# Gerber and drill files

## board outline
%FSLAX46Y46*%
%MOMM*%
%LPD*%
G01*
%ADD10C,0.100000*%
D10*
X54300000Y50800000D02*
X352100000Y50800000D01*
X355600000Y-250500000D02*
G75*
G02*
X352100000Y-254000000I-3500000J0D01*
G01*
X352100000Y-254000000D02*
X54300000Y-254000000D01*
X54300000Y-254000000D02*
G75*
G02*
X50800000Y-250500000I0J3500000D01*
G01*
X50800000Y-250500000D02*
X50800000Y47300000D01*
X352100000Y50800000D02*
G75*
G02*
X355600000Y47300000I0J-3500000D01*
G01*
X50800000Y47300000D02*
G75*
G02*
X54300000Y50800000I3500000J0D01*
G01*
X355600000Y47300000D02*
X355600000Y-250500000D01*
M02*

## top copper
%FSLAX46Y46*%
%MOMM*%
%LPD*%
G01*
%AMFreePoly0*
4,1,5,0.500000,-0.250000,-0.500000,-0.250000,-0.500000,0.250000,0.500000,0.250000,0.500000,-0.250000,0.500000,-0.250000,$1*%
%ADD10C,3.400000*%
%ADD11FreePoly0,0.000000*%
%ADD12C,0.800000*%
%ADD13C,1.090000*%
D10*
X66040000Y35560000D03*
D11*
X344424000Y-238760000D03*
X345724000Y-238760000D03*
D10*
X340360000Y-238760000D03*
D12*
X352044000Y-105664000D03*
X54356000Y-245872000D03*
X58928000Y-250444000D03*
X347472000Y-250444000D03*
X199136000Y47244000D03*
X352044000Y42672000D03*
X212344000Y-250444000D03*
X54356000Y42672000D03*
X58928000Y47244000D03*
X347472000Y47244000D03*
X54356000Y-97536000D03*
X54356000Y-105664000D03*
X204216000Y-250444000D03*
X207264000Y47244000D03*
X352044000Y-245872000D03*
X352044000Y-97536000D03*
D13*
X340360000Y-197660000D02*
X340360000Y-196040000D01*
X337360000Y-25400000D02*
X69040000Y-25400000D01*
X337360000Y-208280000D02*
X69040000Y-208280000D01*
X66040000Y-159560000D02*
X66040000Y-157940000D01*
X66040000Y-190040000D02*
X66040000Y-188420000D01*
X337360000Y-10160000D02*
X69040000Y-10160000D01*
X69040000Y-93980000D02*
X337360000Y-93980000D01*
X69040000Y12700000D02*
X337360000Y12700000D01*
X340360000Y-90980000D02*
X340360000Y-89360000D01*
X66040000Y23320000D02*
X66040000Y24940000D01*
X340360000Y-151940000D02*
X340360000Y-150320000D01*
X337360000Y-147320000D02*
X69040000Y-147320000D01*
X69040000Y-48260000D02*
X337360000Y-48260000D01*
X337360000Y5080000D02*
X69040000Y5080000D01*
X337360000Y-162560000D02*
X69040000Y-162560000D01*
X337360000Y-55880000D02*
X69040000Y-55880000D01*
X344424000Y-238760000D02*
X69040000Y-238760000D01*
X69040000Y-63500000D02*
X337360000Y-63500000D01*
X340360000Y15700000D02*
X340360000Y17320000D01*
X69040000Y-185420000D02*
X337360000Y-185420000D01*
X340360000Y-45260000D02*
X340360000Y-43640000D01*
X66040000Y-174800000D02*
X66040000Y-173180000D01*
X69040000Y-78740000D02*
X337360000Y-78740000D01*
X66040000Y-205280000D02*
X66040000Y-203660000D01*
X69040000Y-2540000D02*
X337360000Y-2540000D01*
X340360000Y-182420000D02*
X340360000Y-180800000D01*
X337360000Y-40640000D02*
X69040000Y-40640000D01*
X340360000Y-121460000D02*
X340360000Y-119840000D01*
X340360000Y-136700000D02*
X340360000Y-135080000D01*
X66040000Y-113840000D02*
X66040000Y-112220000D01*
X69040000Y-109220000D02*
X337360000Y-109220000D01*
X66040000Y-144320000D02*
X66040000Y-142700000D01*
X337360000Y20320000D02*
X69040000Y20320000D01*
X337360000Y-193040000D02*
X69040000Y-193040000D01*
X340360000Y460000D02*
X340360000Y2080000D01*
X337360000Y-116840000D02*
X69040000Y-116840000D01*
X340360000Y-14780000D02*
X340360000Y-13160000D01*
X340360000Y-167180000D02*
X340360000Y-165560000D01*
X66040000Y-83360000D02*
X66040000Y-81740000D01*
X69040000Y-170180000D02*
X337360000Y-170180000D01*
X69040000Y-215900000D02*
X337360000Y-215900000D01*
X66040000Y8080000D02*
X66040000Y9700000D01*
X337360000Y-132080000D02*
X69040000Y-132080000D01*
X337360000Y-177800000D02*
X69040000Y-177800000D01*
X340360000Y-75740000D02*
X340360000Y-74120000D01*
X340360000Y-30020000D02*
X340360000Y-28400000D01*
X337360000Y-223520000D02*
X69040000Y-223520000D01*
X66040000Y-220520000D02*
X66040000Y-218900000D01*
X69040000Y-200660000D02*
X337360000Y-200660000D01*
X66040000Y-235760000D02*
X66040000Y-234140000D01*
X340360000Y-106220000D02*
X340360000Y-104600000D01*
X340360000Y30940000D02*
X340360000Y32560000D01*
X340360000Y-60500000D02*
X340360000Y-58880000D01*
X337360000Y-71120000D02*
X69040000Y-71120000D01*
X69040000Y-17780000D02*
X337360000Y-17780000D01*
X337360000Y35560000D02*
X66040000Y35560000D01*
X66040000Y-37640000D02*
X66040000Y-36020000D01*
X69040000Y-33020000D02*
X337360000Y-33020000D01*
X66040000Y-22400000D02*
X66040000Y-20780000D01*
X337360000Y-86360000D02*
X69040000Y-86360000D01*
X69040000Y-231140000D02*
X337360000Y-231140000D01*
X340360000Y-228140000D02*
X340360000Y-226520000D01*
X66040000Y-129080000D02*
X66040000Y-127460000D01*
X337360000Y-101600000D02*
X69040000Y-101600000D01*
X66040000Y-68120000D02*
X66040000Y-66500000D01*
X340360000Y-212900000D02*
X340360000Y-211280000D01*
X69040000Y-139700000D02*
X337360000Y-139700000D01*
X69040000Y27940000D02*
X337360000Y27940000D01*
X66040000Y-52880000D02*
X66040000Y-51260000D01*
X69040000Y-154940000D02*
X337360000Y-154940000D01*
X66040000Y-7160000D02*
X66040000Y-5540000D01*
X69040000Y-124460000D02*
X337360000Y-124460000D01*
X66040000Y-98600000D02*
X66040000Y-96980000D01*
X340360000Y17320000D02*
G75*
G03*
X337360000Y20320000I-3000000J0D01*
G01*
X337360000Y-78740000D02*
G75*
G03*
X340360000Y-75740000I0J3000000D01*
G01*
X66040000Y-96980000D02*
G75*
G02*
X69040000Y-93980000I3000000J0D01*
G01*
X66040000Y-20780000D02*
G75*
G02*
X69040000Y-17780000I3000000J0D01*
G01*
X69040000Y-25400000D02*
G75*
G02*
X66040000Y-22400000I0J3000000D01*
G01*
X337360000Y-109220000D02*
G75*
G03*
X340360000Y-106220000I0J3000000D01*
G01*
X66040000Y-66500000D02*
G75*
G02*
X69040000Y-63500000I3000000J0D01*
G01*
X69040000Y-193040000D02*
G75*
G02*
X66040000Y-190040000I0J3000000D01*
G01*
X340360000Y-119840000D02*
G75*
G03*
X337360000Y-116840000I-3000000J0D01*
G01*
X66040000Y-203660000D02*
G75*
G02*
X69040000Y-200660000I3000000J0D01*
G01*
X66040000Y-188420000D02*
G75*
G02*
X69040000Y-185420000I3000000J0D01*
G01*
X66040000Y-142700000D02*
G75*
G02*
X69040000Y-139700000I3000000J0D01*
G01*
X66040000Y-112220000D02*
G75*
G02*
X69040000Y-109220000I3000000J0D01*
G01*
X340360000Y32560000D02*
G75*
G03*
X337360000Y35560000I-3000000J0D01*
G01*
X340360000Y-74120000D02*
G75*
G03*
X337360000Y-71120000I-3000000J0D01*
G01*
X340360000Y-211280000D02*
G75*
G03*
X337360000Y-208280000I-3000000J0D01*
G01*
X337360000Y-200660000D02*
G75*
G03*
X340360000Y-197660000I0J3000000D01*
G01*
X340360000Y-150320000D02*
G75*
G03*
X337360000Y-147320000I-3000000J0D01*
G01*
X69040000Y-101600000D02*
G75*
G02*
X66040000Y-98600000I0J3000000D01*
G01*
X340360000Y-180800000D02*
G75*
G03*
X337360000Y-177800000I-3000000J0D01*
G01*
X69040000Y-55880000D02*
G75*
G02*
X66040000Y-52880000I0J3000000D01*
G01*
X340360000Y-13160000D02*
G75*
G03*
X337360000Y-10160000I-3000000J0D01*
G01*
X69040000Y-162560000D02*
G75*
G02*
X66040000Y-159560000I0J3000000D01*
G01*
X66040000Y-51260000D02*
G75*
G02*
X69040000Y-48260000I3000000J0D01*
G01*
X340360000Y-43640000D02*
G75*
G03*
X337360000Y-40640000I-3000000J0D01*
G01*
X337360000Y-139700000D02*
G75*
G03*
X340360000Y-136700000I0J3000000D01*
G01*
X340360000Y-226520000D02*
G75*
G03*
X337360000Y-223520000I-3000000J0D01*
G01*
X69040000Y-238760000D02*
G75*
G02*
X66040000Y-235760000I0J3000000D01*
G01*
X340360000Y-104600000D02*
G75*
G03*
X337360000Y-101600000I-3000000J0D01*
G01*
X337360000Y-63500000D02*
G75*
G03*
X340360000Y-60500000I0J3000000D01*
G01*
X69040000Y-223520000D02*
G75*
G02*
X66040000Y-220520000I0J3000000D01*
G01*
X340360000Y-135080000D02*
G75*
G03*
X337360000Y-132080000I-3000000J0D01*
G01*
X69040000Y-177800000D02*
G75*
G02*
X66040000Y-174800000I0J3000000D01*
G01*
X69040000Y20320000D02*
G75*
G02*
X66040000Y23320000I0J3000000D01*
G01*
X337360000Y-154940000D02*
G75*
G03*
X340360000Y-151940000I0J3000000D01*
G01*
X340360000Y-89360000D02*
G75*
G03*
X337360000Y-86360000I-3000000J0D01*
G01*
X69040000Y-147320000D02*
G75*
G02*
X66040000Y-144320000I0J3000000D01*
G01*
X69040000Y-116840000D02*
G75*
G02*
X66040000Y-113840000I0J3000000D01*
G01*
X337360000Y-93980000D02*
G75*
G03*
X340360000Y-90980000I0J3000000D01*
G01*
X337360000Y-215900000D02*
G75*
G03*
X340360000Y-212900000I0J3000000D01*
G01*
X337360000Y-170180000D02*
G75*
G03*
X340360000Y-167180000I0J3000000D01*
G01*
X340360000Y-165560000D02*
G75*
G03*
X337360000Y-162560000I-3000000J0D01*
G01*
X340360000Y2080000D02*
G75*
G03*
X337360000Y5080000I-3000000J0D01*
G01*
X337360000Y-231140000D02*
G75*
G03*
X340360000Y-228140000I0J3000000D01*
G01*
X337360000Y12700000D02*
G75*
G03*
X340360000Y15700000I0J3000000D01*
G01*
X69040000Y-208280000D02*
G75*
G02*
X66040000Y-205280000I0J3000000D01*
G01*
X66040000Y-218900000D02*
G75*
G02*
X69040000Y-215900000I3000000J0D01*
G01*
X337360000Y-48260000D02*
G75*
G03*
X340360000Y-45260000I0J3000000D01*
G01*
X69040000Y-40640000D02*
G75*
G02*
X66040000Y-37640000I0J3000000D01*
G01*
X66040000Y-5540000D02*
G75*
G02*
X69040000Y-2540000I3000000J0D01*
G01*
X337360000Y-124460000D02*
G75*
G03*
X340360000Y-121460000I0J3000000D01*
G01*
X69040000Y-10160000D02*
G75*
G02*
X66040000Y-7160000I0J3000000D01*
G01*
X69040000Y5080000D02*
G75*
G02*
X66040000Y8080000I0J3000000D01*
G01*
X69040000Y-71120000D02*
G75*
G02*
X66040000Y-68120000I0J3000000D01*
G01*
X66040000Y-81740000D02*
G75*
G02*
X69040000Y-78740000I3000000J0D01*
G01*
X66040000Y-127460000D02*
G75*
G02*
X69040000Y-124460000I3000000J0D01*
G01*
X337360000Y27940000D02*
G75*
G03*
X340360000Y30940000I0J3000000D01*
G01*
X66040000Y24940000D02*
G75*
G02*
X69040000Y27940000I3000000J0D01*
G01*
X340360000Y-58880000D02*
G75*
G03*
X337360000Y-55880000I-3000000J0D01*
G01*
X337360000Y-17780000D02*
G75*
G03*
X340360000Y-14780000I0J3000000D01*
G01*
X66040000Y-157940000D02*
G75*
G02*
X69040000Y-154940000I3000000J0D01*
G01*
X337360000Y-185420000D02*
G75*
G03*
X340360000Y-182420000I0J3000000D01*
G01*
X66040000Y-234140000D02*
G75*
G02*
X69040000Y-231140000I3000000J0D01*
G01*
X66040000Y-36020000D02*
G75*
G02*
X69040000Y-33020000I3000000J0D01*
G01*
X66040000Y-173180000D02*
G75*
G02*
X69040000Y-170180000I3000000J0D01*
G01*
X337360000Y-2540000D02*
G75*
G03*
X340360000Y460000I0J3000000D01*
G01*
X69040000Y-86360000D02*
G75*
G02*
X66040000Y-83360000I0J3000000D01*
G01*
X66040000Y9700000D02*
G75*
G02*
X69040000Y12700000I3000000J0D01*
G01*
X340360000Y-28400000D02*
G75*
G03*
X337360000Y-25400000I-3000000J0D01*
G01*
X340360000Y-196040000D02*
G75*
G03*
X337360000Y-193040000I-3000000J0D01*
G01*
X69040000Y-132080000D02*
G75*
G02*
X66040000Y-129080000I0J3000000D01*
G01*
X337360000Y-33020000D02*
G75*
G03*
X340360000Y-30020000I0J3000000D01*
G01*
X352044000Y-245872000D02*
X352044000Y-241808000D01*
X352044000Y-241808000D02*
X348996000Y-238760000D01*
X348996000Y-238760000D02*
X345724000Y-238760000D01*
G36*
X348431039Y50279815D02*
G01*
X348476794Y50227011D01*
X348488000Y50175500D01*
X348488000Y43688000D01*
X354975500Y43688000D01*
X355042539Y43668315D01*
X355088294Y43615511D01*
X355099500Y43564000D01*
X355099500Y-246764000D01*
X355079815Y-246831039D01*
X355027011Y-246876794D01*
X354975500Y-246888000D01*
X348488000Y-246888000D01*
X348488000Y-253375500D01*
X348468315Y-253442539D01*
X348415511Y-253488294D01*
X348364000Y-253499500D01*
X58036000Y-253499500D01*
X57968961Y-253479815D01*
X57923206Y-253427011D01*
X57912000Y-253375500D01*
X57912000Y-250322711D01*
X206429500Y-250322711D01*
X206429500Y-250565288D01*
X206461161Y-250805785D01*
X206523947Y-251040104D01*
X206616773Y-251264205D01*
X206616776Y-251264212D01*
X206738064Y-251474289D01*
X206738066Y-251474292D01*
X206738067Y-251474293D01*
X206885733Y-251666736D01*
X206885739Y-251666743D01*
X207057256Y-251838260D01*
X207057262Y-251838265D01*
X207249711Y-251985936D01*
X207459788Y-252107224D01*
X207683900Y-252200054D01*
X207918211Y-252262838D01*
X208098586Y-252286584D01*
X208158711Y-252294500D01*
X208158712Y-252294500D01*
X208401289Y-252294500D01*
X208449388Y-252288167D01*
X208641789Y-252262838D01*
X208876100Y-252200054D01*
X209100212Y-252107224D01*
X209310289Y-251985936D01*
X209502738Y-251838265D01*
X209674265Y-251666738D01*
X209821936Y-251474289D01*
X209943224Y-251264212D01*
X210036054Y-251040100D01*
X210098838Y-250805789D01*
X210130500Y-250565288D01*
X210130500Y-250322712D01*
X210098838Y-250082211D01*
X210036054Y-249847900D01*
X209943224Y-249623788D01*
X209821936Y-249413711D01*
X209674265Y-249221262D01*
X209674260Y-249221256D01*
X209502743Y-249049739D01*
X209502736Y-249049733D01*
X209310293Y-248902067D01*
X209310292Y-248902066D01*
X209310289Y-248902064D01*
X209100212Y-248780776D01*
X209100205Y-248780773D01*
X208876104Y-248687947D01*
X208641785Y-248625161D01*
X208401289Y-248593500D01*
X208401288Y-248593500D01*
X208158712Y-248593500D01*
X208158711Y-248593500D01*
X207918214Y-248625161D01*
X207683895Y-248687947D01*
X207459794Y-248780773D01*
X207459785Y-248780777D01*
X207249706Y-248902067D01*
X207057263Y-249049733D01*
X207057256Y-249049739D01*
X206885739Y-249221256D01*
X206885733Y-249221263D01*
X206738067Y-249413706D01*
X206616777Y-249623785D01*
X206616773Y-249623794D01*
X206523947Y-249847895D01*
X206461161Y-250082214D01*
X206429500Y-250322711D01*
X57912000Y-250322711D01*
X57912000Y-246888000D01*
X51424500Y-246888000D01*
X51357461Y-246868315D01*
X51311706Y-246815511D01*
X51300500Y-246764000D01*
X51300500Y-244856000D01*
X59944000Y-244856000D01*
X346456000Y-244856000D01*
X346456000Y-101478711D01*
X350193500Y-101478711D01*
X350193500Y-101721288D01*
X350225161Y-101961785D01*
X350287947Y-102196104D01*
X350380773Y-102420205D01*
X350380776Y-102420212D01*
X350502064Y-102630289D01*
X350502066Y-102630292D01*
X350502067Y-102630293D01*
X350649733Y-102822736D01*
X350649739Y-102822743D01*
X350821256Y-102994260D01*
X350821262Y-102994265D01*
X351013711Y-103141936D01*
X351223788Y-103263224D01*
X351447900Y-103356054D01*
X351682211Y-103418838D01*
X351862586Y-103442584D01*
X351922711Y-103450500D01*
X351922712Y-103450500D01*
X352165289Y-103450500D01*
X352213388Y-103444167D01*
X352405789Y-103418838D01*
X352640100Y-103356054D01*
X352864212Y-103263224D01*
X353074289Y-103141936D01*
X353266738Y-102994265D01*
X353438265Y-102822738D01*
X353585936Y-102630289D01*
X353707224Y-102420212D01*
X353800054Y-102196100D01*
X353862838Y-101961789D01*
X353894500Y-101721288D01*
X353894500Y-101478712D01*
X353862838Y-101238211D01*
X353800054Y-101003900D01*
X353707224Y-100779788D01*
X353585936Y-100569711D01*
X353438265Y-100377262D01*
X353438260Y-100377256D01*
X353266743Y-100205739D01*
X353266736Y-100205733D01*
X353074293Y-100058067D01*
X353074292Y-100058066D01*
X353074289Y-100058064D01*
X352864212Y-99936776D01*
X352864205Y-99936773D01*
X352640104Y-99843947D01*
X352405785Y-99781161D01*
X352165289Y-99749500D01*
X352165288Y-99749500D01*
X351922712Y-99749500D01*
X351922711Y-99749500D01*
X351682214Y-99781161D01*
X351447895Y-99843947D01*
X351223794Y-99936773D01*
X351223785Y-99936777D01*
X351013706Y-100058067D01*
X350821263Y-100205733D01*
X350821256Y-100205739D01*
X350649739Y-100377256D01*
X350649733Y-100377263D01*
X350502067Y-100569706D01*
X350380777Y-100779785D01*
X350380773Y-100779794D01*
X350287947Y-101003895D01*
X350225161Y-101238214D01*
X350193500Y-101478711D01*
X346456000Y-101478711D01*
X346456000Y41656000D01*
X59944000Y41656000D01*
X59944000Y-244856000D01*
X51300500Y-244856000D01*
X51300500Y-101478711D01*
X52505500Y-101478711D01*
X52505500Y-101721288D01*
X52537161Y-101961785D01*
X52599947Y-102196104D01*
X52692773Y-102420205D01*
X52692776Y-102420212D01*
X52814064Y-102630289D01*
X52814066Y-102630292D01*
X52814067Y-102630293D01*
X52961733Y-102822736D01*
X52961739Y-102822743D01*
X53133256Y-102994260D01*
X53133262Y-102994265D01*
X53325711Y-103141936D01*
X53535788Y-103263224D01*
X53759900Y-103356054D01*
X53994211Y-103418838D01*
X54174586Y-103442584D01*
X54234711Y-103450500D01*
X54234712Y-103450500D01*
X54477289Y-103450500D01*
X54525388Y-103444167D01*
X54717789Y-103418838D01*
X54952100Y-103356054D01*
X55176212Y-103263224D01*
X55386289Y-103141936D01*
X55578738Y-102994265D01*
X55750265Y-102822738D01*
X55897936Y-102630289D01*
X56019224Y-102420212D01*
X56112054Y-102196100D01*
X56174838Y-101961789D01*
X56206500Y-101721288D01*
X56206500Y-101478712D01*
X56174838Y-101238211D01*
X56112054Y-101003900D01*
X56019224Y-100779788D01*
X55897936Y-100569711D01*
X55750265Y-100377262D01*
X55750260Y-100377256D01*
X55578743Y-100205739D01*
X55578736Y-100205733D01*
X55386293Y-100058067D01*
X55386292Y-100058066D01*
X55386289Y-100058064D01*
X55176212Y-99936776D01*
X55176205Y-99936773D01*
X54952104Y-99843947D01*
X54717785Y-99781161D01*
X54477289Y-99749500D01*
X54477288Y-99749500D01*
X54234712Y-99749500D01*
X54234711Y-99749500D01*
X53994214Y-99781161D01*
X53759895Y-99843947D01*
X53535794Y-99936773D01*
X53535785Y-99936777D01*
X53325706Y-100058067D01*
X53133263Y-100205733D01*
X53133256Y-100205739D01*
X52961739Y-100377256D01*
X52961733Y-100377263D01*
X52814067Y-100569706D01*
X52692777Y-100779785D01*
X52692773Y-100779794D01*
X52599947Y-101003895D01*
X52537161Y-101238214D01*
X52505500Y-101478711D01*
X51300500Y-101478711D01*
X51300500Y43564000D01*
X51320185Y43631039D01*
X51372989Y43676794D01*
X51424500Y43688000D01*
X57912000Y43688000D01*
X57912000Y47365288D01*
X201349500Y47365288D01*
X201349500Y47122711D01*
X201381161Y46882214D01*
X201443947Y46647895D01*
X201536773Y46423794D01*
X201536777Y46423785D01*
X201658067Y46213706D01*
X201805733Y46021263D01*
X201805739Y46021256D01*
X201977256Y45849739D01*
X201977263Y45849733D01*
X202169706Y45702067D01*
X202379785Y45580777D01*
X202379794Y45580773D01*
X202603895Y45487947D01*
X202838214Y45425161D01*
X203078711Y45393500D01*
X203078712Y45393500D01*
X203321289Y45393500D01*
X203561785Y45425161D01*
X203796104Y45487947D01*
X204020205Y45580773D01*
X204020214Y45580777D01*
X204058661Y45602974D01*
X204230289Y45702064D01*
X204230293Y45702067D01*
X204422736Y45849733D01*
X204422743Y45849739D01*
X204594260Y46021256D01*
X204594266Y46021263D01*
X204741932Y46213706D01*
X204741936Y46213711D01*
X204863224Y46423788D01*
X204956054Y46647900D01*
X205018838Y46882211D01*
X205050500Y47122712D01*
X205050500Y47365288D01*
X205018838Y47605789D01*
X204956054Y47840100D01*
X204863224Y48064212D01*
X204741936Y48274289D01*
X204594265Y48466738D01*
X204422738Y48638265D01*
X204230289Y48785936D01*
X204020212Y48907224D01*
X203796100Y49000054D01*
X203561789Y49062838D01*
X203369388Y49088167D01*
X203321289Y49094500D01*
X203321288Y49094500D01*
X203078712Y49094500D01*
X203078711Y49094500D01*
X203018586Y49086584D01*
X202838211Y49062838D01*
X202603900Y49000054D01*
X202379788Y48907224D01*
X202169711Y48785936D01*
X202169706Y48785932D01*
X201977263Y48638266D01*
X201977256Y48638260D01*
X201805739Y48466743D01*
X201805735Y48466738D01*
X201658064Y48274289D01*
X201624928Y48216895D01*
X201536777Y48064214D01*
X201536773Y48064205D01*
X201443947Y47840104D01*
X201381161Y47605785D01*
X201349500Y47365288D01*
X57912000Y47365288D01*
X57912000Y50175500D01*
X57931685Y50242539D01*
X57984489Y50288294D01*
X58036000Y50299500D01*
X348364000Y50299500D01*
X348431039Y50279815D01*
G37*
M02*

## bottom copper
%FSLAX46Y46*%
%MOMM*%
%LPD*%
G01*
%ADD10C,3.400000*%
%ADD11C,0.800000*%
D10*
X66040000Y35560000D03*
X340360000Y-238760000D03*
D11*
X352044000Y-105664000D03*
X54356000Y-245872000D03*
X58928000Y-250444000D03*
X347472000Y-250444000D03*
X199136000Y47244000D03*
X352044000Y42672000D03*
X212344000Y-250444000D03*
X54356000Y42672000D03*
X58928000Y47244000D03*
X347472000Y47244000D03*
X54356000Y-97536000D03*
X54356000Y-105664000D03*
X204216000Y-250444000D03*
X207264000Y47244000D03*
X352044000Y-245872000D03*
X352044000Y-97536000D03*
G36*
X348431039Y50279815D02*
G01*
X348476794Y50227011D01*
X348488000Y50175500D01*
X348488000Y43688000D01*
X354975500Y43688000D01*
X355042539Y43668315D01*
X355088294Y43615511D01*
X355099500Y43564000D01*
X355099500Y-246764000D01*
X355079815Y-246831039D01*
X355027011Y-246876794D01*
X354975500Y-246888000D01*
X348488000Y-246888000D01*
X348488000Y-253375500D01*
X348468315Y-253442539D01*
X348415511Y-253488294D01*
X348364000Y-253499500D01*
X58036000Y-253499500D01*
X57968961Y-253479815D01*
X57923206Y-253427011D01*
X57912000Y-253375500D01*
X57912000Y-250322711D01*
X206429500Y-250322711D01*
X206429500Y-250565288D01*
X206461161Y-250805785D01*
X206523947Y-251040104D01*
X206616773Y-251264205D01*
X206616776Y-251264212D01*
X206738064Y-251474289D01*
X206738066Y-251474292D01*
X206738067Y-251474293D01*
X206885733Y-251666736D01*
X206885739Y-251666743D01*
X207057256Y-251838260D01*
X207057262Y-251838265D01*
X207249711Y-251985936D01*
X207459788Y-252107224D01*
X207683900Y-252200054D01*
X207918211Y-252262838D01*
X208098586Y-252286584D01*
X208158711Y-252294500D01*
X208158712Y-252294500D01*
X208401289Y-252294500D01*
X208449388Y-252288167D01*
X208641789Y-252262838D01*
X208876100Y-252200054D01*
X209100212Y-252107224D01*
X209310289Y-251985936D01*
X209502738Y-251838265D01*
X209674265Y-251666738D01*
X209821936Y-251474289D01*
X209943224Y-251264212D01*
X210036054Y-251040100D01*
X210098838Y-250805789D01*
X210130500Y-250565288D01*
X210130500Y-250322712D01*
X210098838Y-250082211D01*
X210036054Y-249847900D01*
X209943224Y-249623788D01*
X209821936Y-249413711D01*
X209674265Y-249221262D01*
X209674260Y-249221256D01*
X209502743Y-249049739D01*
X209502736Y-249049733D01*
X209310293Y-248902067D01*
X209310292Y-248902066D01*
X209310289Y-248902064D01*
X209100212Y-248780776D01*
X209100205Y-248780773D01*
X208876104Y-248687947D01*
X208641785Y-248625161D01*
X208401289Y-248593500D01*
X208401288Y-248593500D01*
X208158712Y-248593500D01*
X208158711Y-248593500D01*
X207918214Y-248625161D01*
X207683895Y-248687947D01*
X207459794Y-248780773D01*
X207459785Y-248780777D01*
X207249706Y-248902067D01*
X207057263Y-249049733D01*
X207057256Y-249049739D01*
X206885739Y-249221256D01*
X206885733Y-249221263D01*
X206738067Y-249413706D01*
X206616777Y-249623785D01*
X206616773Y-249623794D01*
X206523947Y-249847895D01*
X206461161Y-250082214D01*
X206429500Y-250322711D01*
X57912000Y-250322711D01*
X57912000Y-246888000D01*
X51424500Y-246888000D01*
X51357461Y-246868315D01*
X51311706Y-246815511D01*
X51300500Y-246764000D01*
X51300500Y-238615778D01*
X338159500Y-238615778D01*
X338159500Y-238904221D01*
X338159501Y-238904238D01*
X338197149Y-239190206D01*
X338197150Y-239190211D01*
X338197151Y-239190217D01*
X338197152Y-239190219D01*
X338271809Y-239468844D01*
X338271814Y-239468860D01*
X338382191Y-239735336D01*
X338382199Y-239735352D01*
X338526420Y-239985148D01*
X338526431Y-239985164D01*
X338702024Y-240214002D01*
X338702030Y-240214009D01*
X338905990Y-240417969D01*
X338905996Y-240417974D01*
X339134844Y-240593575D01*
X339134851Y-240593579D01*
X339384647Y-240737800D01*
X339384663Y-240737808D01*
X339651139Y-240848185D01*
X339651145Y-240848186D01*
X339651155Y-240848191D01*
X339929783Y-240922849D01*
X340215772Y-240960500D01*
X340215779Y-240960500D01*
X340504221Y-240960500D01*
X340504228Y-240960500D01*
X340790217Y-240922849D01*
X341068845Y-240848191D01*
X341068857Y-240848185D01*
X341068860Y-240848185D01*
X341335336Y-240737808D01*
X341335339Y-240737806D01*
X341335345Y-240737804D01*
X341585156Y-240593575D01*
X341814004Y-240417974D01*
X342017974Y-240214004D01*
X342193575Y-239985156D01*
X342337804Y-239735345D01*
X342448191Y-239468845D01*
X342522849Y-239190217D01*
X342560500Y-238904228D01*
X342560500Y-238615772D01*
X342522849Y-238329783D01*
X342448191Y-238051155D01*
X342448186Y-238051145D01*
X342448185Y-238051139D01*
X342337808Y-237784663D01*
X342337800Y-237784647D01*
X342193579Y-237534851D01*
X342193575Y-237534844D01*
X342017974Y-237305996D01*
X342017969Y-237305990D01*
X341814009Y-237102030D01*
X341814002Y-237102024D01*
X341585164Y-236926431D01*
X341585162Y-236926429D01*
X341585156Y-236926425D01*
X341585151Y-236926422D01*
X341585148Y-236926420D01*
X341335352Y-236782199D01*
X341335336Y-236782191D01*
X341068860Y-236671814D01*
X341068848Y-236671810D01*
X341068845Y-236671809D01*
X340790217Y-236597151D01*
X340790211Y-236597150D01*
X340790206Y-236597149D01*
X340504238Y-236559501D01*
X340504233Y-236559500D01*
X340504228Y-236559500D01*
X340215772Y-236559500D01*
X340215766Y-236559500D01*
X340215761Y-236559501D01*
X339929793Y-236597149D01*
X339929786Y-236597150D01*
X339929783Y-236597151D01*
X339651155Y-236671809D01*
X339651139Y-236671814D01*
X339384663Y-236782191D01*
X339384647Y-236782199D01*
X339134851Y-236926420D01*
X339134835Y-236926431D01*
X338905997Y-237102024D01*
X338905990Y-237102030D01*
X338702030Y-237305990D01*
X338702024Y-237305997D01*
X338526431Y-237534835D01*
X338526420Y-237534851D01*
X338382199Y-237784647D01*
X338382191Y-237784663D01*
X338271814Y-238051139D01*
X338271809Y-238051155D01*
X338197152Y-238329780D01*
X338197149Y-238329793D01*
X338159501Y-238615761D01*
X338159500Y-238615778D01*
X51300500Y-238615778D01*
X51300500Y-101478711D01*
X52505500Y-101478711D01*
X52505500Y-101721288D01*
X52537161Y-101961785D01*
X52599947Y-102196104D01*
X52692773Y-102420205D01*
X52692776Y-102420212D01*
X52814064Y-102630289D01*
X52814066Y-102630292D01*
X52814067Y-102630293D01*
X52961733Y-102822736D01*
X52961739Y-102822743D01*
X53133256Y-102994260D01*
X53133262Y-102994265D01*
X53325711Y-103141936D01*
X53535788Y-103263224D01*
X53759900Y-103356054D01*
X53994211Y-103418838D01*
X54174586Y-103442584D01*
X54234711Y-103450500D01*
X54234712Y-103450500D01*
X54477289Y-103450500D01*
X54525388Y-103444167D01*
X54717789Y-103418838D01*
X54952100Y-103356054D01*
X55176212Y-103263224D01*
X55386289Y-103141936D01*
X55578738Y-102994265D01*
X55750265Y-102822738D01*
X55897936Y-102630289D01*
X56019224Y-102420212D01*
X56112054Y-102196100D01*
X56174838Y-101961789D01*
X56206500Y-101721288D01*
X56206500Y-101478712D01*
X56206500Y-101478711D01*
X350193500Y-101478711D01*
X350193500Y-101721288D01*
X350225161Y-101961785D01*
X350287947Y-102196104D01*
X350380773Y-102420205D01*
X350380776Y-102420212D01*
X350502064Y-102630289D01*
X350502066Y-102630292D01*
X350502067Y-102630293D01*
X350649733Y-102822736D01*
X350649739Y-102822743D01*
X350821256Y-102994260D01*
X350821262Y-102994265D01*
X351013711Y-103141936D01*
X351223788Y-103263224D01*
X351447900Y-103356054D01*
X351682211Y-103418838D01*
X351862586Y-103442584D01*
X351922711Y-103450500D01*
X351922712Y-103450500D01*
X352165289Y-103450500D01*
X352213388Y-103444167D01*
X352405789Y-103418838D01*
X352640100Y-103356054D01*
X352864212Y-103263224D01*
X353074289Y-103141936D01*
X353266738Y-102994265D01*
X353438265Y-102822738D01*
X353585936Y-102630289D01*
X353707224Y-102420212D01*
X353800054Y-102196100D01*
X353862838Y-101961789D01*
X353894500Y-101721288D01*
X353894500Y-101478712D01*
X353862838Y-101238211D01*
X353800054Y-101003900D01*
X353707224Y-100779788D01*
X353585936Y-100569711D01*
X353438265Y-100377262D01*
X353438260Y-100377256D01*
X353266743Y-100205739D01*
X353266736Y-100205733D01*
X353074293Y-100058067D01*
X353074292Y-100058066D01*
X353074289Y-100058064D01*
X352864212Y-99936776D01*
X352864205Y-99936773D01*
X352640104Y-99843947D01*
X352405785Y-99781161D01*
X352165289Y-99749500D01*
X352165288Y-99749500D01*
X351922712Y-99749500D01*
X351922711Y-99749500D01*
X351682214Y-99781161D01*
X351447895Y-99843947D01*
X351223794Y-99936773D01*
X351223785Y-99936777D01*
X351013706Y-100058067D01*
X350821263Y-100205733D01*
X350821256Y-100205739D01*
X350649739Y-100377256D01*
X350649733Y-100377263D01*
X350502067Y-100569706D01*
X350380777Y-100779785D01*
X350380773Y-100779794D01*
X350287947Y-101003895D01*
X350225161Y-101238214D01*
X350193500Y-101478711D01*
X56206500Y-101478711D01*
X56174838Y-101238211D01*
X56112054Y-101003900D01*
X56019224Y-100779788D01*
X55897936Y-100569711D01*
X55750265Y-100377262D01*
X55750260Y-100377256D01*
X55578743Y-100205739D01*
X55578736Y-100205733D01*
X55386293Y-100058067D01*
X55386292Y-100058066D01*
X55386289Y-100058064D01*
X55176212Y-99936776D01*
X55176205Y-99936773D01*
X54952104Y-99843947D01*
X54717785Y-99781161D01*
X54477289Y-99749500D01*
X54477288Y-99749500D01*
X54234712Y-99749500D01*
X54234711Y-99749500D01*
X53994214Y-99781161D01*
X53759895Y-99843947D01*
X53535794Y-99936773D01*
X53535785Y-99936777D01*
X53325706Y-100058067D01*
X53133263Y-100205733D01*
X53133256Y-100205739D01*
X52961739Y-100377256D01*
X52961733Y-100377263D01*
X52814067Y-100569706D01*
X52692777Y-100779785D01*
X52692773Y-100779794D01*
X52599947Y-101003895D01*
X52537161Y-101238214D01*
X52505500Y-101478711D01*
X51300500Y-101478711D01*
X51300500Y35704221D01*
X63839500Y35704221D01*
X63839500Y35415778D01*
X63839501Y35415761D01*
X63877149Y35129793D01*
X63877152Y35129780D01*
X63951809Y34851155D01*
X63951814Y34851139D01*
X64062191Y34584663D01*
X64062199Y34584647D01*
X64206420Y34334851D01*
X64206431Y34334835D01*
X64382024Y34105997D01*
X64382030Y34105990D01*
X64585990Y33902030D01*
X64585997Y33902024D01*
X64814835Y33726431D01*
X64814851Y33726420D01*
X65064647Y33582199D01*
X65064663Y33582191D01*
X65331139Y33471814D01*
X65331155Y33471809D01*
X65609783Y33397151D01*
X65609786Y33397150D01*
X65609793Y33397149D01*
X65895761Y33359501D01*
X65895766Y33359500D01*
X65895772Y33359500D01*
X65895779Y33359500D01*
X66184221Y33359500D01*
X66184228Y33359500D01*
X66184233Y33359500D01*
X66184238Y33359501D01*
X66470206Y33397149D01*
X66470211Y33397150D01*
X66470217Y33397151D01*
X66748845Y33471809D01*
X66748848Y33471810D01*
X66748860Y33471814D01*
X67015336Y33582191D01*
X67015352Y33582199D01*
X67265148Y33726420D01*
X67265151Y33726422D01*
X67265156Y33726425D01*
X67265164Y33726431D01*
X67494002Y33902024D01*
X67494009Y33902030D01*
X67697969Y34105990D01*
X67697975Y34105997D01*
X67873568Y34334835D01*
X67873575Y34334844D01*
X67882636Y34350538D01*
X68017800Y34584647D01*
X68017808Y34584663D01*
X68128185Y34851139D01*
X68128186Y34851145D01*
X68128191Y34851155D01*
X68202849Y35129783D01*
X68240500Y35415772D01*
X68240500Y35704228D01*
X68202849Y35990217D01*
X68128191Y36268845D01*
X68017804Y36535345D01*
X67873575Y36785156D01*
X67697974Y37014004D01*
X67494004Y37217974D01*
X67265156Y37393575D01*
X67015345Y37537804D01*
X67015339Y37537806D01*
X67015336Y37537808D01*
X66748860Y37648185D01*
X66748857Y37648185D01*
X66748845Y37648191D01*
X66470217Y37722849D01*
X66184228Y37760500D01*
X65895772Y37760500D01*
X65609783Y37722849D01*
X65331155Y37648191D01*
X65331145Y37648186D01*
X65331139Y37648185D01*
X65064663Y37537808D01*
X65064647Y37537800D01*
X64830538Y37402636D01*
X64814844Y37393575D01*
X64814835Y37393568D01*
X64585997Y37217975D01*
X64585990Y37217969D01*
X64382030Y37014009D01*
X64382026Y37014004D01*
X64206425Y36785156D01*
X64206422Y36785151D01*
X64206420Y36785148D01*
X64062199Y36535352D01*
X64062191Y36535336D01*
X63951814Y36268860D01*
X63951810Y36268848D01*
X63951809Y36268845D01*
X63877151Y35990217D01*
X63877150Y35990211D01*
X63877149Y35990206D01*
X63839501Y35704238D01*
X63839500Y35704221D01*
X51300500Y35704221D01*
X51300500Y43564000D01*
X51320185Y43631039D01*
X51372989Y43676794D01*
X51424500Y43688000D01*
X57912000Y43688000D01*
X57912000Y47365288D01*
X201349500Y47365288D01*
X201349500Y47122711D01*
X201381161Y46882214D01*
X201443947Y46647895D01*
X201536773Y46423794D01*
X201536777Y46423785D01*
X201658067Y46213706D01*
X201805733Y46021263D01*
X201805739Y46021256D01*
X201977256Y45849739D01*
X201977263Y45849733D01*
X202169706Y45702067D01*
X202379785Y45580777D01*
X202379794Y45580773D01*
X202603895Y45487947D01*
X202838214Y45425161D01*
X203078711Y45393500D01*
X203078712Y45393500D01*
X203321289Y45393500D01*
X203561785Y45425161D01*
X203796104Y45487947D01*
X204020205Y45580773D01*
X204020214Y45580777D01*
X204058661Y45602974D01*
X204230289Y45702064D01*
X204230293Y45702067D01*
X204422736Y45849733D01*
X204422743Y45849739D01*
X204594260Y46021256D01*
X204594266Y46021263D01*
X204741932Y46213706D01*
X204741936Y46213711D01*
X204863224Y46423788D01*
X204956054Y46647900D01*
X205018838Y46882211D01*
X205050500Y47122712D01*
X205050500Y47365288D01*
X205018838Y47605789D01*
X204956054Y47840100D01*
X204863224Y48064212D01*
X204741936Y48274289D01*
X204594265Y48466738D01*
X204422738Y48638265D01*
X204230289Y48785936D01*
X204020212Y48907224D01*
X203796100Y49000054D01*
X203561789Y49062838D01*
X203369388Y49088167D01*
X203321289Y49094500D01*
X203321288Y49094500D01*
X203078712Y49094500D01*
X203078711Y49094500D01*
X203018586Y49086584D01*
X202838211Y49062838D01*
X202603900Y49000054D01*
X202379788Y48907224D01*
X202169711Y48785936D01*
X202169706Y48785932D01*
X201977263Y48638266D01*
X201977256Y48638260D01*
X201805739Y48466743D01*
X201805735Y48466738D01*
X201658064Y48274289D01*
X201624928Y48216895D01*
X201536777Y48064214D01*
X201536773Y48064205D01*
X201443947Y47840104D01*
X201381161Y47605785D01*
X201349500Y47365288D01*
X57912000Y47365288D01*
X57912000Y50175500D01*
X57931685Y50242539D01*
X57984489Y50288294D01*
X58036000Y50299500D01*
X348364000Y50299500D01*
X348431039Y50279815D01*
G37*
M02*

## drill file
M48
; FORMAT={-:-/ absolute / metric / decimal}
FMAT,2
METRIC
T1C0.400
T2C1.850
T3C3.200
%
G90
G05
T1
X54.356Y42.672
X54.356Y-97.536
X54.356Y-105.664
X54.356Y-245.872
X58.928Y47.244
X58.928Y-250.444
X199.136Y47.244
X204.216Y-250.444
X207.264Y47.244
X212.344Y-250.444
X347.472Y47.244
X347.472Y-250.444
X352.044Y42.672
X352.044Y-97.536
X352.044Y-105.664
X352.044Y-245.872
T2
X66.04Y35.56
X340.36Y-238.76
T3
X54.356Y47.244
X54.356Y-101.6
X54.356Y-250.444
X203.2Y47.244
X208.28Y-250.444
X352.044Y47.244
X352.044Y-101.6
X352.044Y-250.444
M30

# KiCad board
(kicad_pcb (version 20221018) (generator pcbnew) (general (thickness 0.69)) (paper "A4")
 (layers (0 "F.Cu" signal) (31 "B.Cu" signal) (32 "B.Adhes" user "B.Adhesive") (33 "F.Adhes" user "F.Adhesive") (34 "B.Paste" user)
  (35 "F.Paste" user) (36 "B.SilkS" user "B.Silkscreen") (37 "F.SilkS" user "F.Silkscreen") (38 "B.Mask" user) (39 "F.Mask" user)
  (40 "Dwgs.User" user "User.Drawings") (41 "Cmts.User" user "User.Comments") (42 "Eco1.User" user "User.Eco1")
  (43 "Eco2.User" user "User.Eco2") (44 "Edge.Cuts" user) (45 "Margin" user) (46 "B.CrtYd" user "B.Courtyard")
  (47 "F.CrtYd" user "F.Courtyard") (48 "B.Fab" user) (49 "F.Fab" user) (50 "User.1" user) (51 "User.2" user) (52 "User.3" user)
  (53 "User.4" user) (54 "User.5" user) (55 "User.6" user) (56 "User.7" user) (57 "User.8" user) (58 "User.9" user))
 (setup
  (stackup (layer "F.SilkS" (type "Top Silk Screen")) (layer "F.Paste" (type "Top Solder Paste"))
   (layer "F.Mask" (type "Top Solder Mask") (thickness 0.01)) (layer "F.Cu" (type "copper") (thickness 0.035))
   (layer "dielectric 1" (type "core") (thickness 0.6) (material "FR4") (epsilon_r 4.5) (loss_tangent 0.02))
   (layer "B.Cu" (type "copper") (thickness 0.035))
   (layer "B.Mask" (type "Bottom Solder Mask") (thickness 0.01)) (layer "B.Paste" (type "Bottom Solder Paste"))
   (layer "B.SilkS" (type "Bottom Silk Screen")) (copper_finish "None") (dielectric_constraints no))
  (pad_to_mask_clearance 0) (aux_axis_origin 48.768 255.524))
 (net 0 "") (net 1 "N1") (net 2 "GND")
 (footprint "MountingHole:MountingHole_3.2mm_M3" (layer "F.Cu") (at 203.2 -47.244)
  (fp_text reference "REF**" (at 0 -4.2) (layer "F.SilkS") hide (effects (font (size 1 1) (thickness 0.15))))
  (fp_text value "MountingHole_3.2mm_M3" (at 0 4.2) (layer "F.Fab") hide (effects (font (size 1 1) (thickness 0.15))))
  (pad "" np_thru_hole circle (at 0 0) (size 3.2 3.2) (drill 3.2) (layers "F&B.Cu" "*.Mask")))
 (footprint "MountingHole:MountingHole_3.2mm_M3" (layer "F.Cu") (at 208.28 250.444)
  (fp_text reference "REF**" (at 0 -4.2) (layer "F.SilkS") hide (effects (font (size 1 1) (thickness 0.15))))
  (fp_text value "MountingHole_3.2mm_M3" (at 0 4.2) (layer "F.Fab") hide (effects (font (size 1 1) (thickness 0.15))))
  (pad "" np_thru_hole circle (at 0 0) (size 3.2 3.2) (drill 3.2) (layers "F&B.Cu" "*.Mask")))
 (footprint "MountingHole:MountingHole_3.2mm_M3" (layer "F.Cu") (at 54.356 101.6)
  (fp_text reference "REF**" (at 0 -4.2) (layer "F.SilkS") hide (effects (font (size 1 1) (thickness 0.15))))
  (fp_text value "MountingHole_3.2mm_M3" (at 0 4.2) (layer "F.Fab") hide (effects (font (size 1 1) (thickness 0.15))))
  (pad "" np_thru_hole circle (at 0 0) (size 3.2 3.2) (drill 3.2) (layers "F&B.Cu" "*.Mask")))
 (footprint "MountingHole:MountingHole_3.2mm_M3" (layer "F.Cu") (at 352.044 250.444)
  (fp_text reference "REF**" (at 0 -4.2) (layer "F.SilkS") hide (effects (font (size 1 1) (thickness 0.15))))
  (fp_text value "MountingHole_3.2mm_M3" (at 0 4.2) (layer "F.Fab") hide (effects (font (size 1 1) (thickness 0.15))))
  (pad "" np_thru_hole circle (at 0 0) (size 3.2 3.2) (drill 3.2) (layers "F&B.Cu" "*.Mask")))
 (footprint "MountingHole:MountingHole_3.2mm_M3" (layer "F.Cu") (at 54.356 250.444)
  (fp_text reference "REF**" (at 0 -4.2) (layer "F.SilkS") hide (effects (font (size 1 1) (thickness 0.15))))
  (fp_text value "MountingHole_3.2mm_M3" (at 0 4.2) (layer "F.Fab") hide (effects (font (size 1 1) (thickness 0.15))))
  (pad "" np_thru_hole circle (at 0 0) (size 3.2 3.2) (drill 3.2) (layers "F&B.Cu" "*.Mask")))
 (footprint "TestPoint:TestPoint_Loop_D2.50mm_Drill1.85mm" (layer "F.Cu") (at 66.04 -35.56)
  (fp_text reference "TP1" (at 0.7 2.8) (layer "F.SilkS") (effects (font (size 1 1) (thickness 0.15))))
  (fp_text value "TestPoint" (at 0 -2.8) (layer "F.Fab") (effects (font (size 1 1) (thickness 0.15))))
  (pad "1" thru_hole circle (at 0 0) (size 3.4 3.4) (drill 1.85) (layers "*.Cu" "*.Mask") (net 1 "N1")))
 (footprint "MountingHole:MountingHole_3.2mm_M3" (layer "F.Cu") (at 352.044 -47.244)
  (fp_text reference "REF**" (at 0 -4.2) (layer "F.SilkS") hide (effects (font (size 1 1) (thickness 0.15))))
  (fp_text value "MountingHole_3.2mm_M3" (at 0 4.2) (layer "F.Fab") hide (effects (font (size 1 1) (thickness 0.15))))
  (pad "" np_thru_hole circle (at 0 0) (size 3.2 3.2) (drill 3.2) (layers "F&B.Cu" "*.Mask")))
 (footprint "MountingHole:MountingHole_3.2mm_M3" (layer "F.Cu") (at 54.356 -47.244)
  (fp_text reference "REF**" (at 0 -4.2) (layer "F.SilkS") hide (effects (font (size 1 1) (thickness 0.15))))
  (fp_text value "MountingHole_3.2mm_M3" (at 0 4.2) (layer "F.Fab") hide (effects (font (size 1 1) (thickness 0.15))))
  (pad "" np_thru_hole circle (at 0 0) (size 3.2 3.2) (drill 3.2) (layers "*.Cu" "*.Mask")))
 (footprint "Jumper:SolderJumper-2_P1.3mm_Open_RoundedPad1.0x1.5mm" (layer "F.Cu") (at 345.074 238.76)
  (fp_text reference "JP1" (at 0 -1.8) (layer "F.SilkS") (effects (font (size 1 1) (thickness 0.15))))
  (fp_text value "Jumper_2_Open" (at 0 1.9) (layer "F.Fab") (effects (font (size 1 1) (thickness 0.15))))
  (pad "1" smd custom (at -0.65 0) (size 1 0.5) (layers "F.Cu" "F.Mask") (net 1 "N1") (zone_connect 2) (thermal_bridge_angle 45)
   (options (clearance outline) (anchor rect)) (primitives))
  (pad "2" smd custom (at 0.65 0) (size 1 0.5) (layers "F.Cu" "F.Mask") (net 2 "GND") (zone_connect 2) (thermal_bridge_angle 45)
   (options (clearance outline) (anchor rect)) (primitives)))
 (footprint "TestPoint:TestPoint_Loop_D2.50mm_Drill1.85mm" (layer "F.Cu") (at 340.36 238.76)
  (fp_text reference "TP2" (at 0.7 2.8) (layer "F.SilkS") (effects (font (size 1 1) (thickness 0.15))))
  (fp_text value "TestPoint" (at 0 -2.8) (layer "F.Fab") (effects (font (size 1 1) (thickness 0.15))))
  (pad "1" thru_hole circle (at 0 0) (size 3.4 3.4) (drill 1.85) (layers "*.Cu" "*.Mask") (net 1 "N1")))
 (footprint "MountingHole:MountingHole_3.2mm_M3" (layer "F.Cu") (at 352.044 101.6)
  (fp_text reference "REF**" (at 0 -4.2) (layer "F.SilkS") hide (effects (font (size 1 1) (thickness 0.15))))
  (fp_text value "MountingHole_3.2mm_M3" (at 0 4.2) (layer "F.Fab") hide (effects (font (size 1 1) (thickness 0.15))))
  (pad "" np_thru_hole circle (at 0 0) (size 3.2 3.2) (drill 3.2) (layers "F&B.Cu" "*.Mask")))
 (gr_line (start 54.3 -50.8) (end 352.1 -50.8) (stroke (width 0.1) (type default)) (layer "Edge.Cuts"))
 (gr_arc (start 355.6 250.5) (mid 354.574874 252.974874) (end 352.1 254) (stroke (width 0.1) (type default)) (layer "Edge.Cuts"))
 (gr_line (start 352.1 254) (end 54.3 254) (stroke (width 0.1) (type default)) (layer "Edge.Cuts"))
 (gr_arc (start 54.3 254) (mid 51.825126 252.974874) (end 50.8 250.5) (stroke (width 0.1) (type default)) (layer "Edge.Cuts"))
 (gr_line (start 50.8 250.5) (end 50.8 -47.3) (stroke (width 0.1) (type default)) (layer "Edge.Cuts"))
 (gr_arc (start 352.1 -50.8) (mid 354.574874 -49.774874) (end 355.6 -47.3) (stroke (width 0.1) (type default)) (layer "Edge.Cuts"))
 (gr_arc (start 50.8 -47.3) (mid 51.825126 -49.774874) (end 54.3 -50.8) (stroke (width 0.1) (type default)) (layer "Edge.Cuts"))
 (gr_line (start 355.6 -47.3) (end 355.6 250.5) (stroke (width 0.1) (type default)) (layer "Edge.Cuts"))
 (segment (start 340.36 197.66) (end 340.36 196.04) (width 1.09) (layer "F.Cu") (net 1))
 (segment (start 337.36 25.4) (end 69.04 25.4) (width 1.09) (layer "F.Cu") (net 1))
 (segment (start 337.36 208.28) (end 69.04 208.28) (width 1.09) (layer "F.Cu") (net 1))
 (segment (start 66.04 159.56) (end 66.04 157.94) (width 1.09) (layer "F.Cu") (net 1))
 (segment (start 66.04 190.04) (end 66.04 188.42) (width 1.09) (layer "F.Cu") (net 1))
 (segment (start 337.36 10.16) (end 69.04 10.16) (width 1.09) (layer "F.Cu") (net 1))
 (segment (start 69.04 93.98) (end 337.36 93.98) (width 1.09) (layer "F.Cu") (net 1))
 (segment (start 69.04 -12.7) (end 337.36 -12.7) (width 1.09) (layer "F.Cu") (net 1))
 (segment (start 340.36 90.98) (end 340.36 89.36) (width 1.09) (layer "F.Cu") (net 1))
 (segment (start 66.04 -23.32) (end 66.04 -24.94) (width 1.09) (layer "F.Cu") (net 1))
 (segment (start 340.36 151.94) (end 340.36 150.32) (width 1.09) (layer "F.Cu") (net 1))
 (segment (start 337.36 147.32) (end 69.04 147.32) (width 1.09) (layer "F.Cu") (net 1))
 (segment (start 69.04 48.26) (end 337.36 48.26) (width 1.09) (layer "F.Cu") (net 1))
 (segment (start 337.36 -5.08) (end 69.04 -5.08) (width 1.09) (layer "F.Cu") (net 1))
 (segment (start 337.36 162.56) (end 69.04 162.56) (width 1.09) (layer "F.Cu") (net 1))
 (segment (start 337.36 55.88) (end 69.04 55.88) (width 1.09) (layer "F.Cu") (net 1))
 (segment (start 344.424 238.76) (end 69.04 238.76) (width 1.09) (layer "F.Cu") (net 1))
 (segment (start 69.04 63.5) (end 337.36 63.5) (width 1.09) (layer "F.Cu") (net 1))
 (segment (start 340.36 -15.7) (end 340.36 -17.32) (width 1.09) (layer "F.Cu") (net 1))
 (segment (start 69.04 185.42) (end 337.36 185.42) (width 1.09) (layer "F.Cu") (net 1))
 (segment (start 340.36 45.26) (end 340.36 43.64) (width 1.09) (layer "F.Cu") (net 1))
 (segment (start 66.04 174.8) (end 66.04 173.18) (width 1.09) (layer "F.Cu") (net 1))
 (segment (start 69.04 78.74) (end 337.36 78.74) (width 1.09) (layer "F.Cu") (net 1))
 (segment (start 66.04 205.28) (end 66.04 203.66) (width 1.09) (layer "F.Cu") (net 1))
 (segment (start 69.04 2.54) (end 337.36 2.54) (width 1.09) (layer "F.Cu") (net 1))
 (segment (start 340.36 182.42) (end 340.36 180.8) (width 1.09) (layer "F.Cu") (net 1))
 (segment (start 337.36 40.64) (end 69.04 40.64) (width 1.09) (layer "F.Cu") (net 1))
 (segment (start 340.36 121.46) (end 340.36 119.84) (width 1.09) (layer "F.Cu") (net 1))
 (segment (start 340.36 136.7) (end 340.36 135.08) (width 1.09) (layer "F.Cu") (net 1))
 (segment (start 66.04 113.84) (end 66.04 112.22) (width 1.09) (layer "F.Cu") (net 1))
 (segment (start 69.04 109.22) (end 337.36 109.22) (width 1.09) (layer "F.Cu") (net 1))
 (segment (start 66.04 144.32) (end 66.04 142.7) (width 1.09) (layer "F.Cu") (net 1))
 (segment (start 337.36 -20.32) (end 69.04 -20.32) (width 1.09) (layer "F.Cu") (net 1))
 (segment (start 337.36 193.04) (end 69.04 193.04) (width 1.09) (layer "F.Cu") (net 1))
 (segment (start 340.36 -0.46) (end 340.36 -2.08) (width 1.09) (layer "F.Cu") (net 1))
 (segment (start 337.36 116.84) (end 69.04 116.84) (width 1.09) (layer "F.Cu") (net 1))
 (segment (start 340.36 14.78) (end 340.36 13.16) (width 1.09) (layer "F.Cu") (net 1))
 (segment (start 340.36 167.18) (end 340.36 165.56) (width 1.09) (layer "F.Cu") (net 1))
 (segment (start 66.04 83.36) (end 66.04 81.74) (width 1.09) (layer "F.Cu") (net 1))
 (segment (start 69.04 170.18) (end 337.36 170.18) (width 1.09) (layer "F.Cu") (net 1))
 (segment (start 69.04 215.9) (end 337.36 215.9) (width 1.09) (layer "F.Cu") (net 1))
 (segment (start 66.04 -8.08) (end 66.04 -9.7) (width 1.09) (layer "F.Cu") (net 1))
 (segment (start 337.36 132.08) (end 69.04 132.08) (width 1.09) (layer "F.Cu") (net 1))
 (segment (start 337.36 177.8) (end 69.04 177.8) (width 1.09) (layer "F.Cu") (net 1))
 (segment (start 340.36 75.74) (end 340.36 74.12) (width 1.09) (layer "F.Cu") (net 1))
 (segment (start 340.36 30.02) (end 340.36 28.4) (width 1.09) (layer "F.Cu") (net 1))
 (segment (start 337.36 223.52) (end 69.04 223.52) (width 1.09) (layer "F.Cu") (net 1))
 (segment (start 66.04 220.52) (end 66.04 218.9) (width 1.09) (layer "F.Cu") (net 1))
 (segment (start 69.04 200.66) (end 337.36 200.66) (width 1.09) (layer "F.Cu") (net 1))
 (segment (start 66.04 235.76) (end 66.04 234.14) (width 1.09) (layer "F.Cu") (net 1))
 (segment (start 340.36 106.22) (end 340.36 104.6) (width 1.09) (layer "F.Cu") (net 1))
 (segment (start 340.36 -30.94) (end 340.36 -32.56) (width 1.09) (layer "F.Cu") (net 1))
 (segment (start 340.36 60.5) (end 340.36 58.88) (width 1.09) (layer "F.Cu") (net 1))
 (segment (start 337.36 71.12) (end 69.04 71.12) (width 1.09) (layer "F.Cu") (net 1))
 (segment (start 69.04 17.78) (end 337.36 17.78) (width 1.09) (layer "F.Cu") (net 1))
 (segment (start 337.36 -35.56) (end 66.04 -35.56) (width 1.09) (layer "F.Cu") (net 1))
 (segment (start 66.04 37.64) (end 66.04 36.02) (width 1.09) (layer "F.Cu") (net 1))
 (segment (start 69.04 33.02) (end 337.36 33.02) (width 1.09) (layer "F.Cu") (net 1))
 (segment (start 66.04 22.4) (end 66.04 20.78) (width 1.09) (layer "F.Cu") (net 1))
 (segment (start 337.36 86.36) (end 69.04 86.36) (width 1.09) (layer "F.Cu") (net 1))
 (segment (start 69.04 231.14) (end 337.36 231.14) (width 1.09) (layer "F.Cu") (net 1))
 (segment (start 340.36 228.14) (end 340.36 226.52) (width 1.09) (layer "F.Cu") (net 1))
 (segment (start 66.04 129.08) (end 66.04 127.46) (width 1.09) (layer "F.Cu") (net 1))
 (segment (start 337.36 101.6) (end 69.04 101.6) (width 1.09) (layer "F.Cu") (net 1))
 (segment (start 66.04 68.12) (end 66.04 66.5) (width 1.09) (layer "F.Cu") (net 1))
 (segment (start 340.36 212.9) (end 340.36 211.28) (width 1.09) (layer "F.Cu") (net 1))
 (segment (start 69.04 139.7) (end 337.36 139.7) (width 1.09) (layer "F.Cu") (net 1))
 (segment (start 69.04 -27.94) (end 337.36 -27.94) (width 1.09) (layer "F.Cu") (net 1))
 (segment (start 66.04 52.88) (end 66.04 51.26) (width 1.09) (layer "F.Cu") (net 1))
 (segment (start 69.04 154.94) (end 337.36 154.94) (width 1.09) (layer "F.Cu") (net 1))
 (segment (start 66.04 7.16) (end 66.04 5.54) (width 1.09) (layer "F.Cu") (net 1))
 (segment (start 69.04 124.46) (end 337.36 124.46) (width 1.09) (layer "F.Cu") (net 1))
 (segment (start 66.04 98.6) (end 66.04 96.98) (width 1.09) (layer "F.Cu") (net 1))
 (arc (start 340.36 -17.32) (mid 339.48132 -19.44132) (end 337.36 -20.32) (width 1.09) (layer "F.Cu") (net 1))
 (arc (start 337.36 78.74) (mid 339.48132 77.86132) (end 340.36 75.74) (width 1.09) (layer "F.Cu") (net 1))
 (arc (start 66.04 96.98) (mid 66.91868 94.85868) (end 69.04 93.98) (width 1.09) (layer "F.Cu") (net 1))
 (arc (start 66.04 20.78) (mid 66.91868 18.65868) (end 69.04 17.78) (width 1.09) (layer "F.Cu") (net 1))
 (arc (start 69.04 25.4) (mid 66.91868 24.52132) (end 66.04 22.4) (width 1.09) (layer "F.Cu") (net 1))
 (arc (start 337.36 109.22) (mid 339.48132 108.34132) (end 340.36 106.22) (width 1.09) (layer "F.Cu") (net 1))
 (arc (start 66.04 66.5) (mid 66.91868 64.37868) (end 69.04 63.5) (width 1.09) (layer "F.Cu") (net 1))
 (arc (start 69.04 193.04) (mid 66.91868 192.16132) (end 66.04 190.04) (width 1.09) (layer "F.Cu") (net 1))
 (arc (start 340.36 119.84) (mid 339.48132 117.71868) (end 337.36 116.84) (width 1.09) (layer "F.Cu") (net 1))
 (arc (start 66.04 203.66) (mid 66.91868 201.53868) (end 69.04 200.66) (width 1.09) (layer "F.Cu") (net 1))
 (arc (start 66.04 188.42) (mid 66.91868 186.29868) (end 69.04 185.42) (width 1.09) (layer "F.Cu") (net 1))
 (arc (start 66.04 142.7) (mid 66.91868 140.57868) (end 69.04 139.7) (width 1.09) (layer "F.Cu") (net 1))
 (arc (start 66.04 112.22) (mid 66.91868 110.09868) (end 69.04 109.22) (width 1.09) (layer "F.Cu") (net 1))
 (arc (start 340.36 -32.56) (mid 339.48132 -34.68132) (end 337.36 -35.56) (width 1.09) (layer "F.Cu") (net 1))
 (arc (start 340.36 74.12) (mid 339.48132 71.99868) (end 337.36 71.12) (width 1.09) (layer "F.Cu") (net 1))
 (arc (start 340.36 211.28) (mid 339.48132 209.15868) (end 337.36 208.28) (width 1.09) (layer "F.Cu") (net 1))
 (arc (start 337.36 200.66) (mid 339.48132 199.78132) (end 340.36 197.66) (width 1.09) (layer "F.Cu") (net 1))
 (arc (start 340.36 150.32) (mid 339.48132 148.19868) (end 337.36 147.32) (width 1.09) (layer "F.Cu") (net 1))
 (arc (start 69.04 101.6) (mid 66.91868 100.72132) (end 66.04 98.6) (width 1.09) (layer "F.Cu") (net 1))
 (arc (start 340.36 180.8) (mid 339.48132 178.67868) (end 337.36 177.8) (width 1.09) (layer "F.Cu") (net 1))
 (arc (start 69.04 55.88) (mid 66.91868 55.00132) (end 66.04 52.88) (width 1.09) (layer "F.Cu") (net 1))
 (arc (start 340.36 13.16) (mid 339.48132 11.03868) (end 337.36 10.16) (width 1.09) (layer "F.Cu") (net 1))
 (arc (start 69.04 162.56) (mid 66.91868 161.68132) (end 66.04 159.56) (width 1.09) (layer "F.Cu") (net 1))
 (arc (start 66.04 51.26) (mid 66.91868 49.13868) (end 69.04 48.26) (width 1.09) (layer "F.Cu") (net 1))
 (arc (start 340.36 43.64) (mid 339.48132 41.51868) (end 337.36 40.64) (width 1.09) (layer "F.Cu") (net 1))
 (arc (start 337.36 139.7) (mid 339.48132 138.82132) (end 340.36 136.7) (width 1.09) (layer "F.Cu") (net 1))
 (arc (start 340.36 226.52) (mid 339.48132 224.39868) (end 337.36 223.52) (width 1.09) (layer "F.Cu") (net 1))
 (arc (start 69.04 238.76) (mid 66.91868 237.88132) (end 66.04 235.76) (width 1.09) (layer "F.Cu") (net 1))
 (arc (start 340.36 104.6) (mid 339.48132 102.47868) (end 337.36 101.6) (width 1.09) (layer "F.Cu") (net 1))
 (arc (start 337.36 63.5) (mid 339.48132 62.62132) (end 340.36 60.5) (width 1.09) (layer "F.Cu") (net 1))
 (arc (start 69.04 223.52) (mid 66.91868 222.64132) (end 66.04 220.52) (width 1.09) (layer "F.Cu") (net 1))
 (arc (start 340.36 135.08) (mid 339.48132 132.95868) (end 337.36 132.08) (width 1.09) (layer "F.Cu") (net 1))
 (arc (start 69.04 177.8) (mid 66.91868 176.92132) (end 66.04 174.8) (width 1.09) (layer "F.Cu") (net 1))
 (arc (start 69.04 -20.32) (mid 66.91868 -21.19868) (end 66.04 -23.32) (width 1.09) (layer "F.Cu") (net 1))
 (arc (start 337.36 154.94) (mid 339.48132 154.06132) (end 340.36 151.94) (width 1.09) (layer "F.Cu") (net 1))
 (arc (start 340.36 89.36) (mid 339.48132 87.23868) (end 337.36 86.36) (width 1.09) (layer "F.Cu") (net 1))
 (arc (start 69.04 147.32) (mid 66.91868 146.44132) (end 66.04 144.32) (width 1.09) (layer "F.Cu") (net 1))
 (arc (start 69.04 116.84) (mid 66.91868 115.96132) (end 66.04 113.84) (width 1.09) (layer "F.Cu") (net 1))
 (arc (start 337.36 93.98) (mid 339.48132 93.10132) (end 340.36 90.98) (width 1.09) (layer "F.Cu") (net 1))
 (arc (start 337.36 215.9) (mid 339.48132 215.02132) (end 340.36 212.9) (width 1.09) (layer "F.Cu") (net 1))
 (arc (start 337.36 170.18) (mid 339.48132 169.30132) (end 340.36 167.18) (width 1.09) (layer "F.Cu") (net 1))
 (arc (start 340.36 165.56) (mid 339.48132 163.43868) (end 337.36 162.56) (width 1.09) (layer "F.Cu") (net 1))
 (arc (start 340.36 -2.08) (mid 339.48132 -4.20132) (end 337.36 -5.08) (width 1.09) (layer "F.Cu") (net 1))
 (arc (start 337.36 231.14) (mid 339.48132 230.26132) (end 340.36 228.14) (width 1.09) (layer "F.Cu") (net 1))
 (arc (start 337.36 -12.7) (mid 339.48132 -13.57868) (end 340.36 -15.7) (width 1.09) (layer "F.Cu") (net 1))
 (arc (start 69.04 208.28) (mid 66.91868 207.40132) (end 66.04 205.28) (width 1.09) (layer "F.Cu") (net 1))
 (arc (start 66.04 218.9) (mid 66.91868 216.77868) (end 69.04 215.9) (width 1.09) (layer "F.Cu") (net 1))
 (arc (start 337.36 48.26) (mid 339.48132 47.38132) (end 340.36 45.26) (width 1.09) (layer "F.Cu") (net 1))
 (arc (start 69.04 40.64) (mid 66.91868 39.76132) (end 66.04 37.64) (width 1.09) (layer "F.Cu") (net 1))
 (arc (start 66.04 5.54) (mid 66.91868 3.41868) (end 69.04 2.54) (width 1.09) (layer "F.Cu") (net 1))
 (arc (start 337.36 124.46) (mid 339.48132 123.58132) (end 340.36 121.46) (width 1.09) (layer "F.Cu") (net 1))
 (arc (start 69.04 10.16) (mid 66.91868 9.28132) (end 66.04 7.16) (width 1.09) (layer "F.Cu") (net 1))
 (arc (start 69.04 -5.08) (mid 66.91868 -5.95868) (end 66.04 -8.08) (width 1.09) (layer "F.Cu") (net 1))
 (arc (start 69.04 71.12) (mid 66.91868 70.24132) (end 66.04 68.12) (width 1.09) (layer "F.Cu") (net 1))
 (arc (start 66.04 81.74) (mid 66.91868 79.61868) (end 69.04 78.74) (width 1.09) (layer "F.Cu") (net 1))
 (arc (start 66.04 127.46) (mid 66.91868 125.33868) (end 69.04 124.46) (width 1.09) (layer "F.Cu") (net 1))
 (arc (start 337.36 -27.94) (mid 339.48132 -28.81868) (end 340.36 -30.94) (width 1.09) (layer "F.Cu") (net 1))
 (arc (start 66.04 -24.94) (mid 66.91868 -27.06132) (end 69.04 -27.94) (width 1.09) (layer "F.Cu") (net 1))
 (arc (start 340.36 58.88) (mid 339.48132 56.75868) (end 337.36 55.88) (width 1.09) (layer "F.Cu") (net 1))
 (arc (start 337.36 17.78) (mid 339.48132 16.90132) (end 340.36 14.78) (width 1.09) (layer "F.Cu") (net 1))
 (arc (start 66.04 157.94) (mid 66.91868 155.81868) (end 69.04 154.94) (width 1.09) (layer "F.Cu") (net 1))
 (arc (start 337.36 185.42) (mid 339.48132 184.54132) (end 340.36 182.42) (width 1.09) (layer "F.Cu") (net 1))
 (arc (start 66.04 234.14) (mid 66.91868 232.01868) (end 69.04 231.14) (width 1.09) (layer "F.Cu") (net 1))
 (arc (start 66.04 36.02) (mid 66.91868 33.89868) (end 69.04 33.02) (width 1.09) (layer "F.Cu") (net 1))
 (arc (start 66.04 173.18) (mid 66.91868 171.05868) (end 69.04 170.18) (width 1.09) (layer "F.Cu") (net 1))
 (arc (start 337.36 2.54) (mid 339.48132 1.66132) (end 340.36 -0.46) (width 1.09) (layer "F.Cu") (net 1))
 (arc (start 69.04 86.36) (mid 66.91868 85.48132) (end 66.04 83.36) (width 1.09) (layer "F.Cu") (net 1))
 (arc (start 66.04 -9.7) (mid 66.91868 -11.82132) (end 69.04 -12.7) (width 1.09) (layer "F.Cu") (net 1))
 (arc (start 340.36 28.4) (mid 339.48132 26.27868) (end 337.36 25.4) (width 1.09) (layer "F.Cu") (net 1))
 (arc (start 340.36 196.04) (mid 339.48132 193.91868) (end 337.36 193.04) (width 1.09) (layer "F.Cu") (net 1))
 (arc (start 69.04 132.08) (mid 66.91868 131.20132) (end 66.04 129.08) (width 1.09) (layer "F.Cu") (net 1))
 (arc (start 337.36 33.02) (mid 339.48132 32.14132) (end 340.36 30.02) (width 1.09) (layer "F.Cu") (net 1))
 (segment (start 352.044 245.872) (end 352.044 241.808) (width 1.09) (layer "F.Cu") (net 2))
 (segment (start 352.044 241.808) (end 348.996 238.76) (width 1.09) (layer "F.Cu") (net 2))
 (segment (start 348.996 238.76) (end 345.724 238.76) (width 1.09) (layer "F.Cu") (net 2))
 (via (at 352.044 105.664) (size 0.8) (drill 0.4) (layers "F.Cu" "B.Cu") (free) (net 2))
 (via (at 54.356 245.872) (size 0.8) (drill 0.4) (layers "F.Cu" "B.Cu") (free) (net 2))
 (via (at 58.928 250.444) (size 0.8) (drill 0.4) (layers "F.Cu" "B.Cu") (free) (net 2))
 (via (at 347.472 250.444) (size 0.8) (drill 0.4) (layers "F.Cu" "B.Cu") (free) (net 2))
 (via (at 199.136 -47.244) (size 0.8) (drill 0.4) (layers "F.Cu" "B.Cu") (free) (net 2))
 (via (at 352.044 -42.672) (size 0.8) (drill 0.4) (layers "F.Cu" "B.Cu") (free) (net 2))
 (via (at 212.344 250.444) (size 0.8) (drill 0.4) (layers "F.Cu" "B.Cu") (free) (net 2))
 (via (at 54.356 -42.672) (size 0.8) (drill 0.4) (layers "F.Cu" "B.Cu") (free) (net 2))
 (via (at 58.928 -47.244) (size 0.8) (drill 0.4) (layers "F.Cu" "B.Cu") (free) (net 2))
 (via (at 347.472 -47.244) (size 0.8) (drill 0.4) (layers "F.Cu" "B.Cu") (free) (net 2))
 (via (at 54.356 97.536) (size 0.8) (drill 0.4) (layers "F.Cu" "B.Cu") (free) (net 2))
 (via (at 54.356 105.664) (size 0.8) (drill 0.4) (layers "F.Cu" "B.Cu") (free) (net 2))
 (via (at 204.216 250.444) (size 0.8) (drill 0.4) (layers "F.Cu" "B.Cu") (free) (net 2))
 (via (at 207.264 -47.244) (size 0.8) (drill 0.4) (layers "F.Cu" "B.Cu") (free) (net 2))
 (via (at 352.044 245.872) (size 0.8) (drill 0.4) (layers "F.Cu" "B.Cu") (free) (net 2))
 (via (at 352.044 97.536) (size 0.8) (drill 0.4) (layers "F.Cu" "B.Cu") (free) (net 2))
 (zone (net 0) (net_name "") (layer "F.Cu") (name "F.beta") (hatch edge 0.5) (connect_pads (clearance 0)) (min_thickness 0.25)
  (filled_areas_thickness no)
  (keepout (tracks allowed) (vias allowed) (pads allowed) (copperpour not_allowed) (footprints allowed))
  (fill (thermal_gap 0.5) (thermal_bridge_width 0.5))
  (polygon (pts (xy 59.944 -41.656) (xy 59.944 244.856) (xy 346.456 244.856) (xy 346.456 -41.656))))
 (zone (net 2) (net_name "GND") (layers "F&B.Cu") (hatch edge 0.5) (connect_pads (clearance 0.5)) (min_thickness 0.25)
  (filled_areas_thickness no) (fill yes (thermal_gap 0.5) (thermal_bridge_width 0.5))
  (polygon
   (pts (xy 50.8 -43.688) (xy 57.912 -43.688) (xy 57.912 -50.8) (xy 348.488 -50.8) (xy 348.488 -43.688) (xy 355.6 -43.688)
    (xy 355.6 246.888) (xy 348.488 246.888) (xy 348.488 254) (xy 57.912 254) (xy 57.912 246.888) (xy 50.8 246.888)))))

